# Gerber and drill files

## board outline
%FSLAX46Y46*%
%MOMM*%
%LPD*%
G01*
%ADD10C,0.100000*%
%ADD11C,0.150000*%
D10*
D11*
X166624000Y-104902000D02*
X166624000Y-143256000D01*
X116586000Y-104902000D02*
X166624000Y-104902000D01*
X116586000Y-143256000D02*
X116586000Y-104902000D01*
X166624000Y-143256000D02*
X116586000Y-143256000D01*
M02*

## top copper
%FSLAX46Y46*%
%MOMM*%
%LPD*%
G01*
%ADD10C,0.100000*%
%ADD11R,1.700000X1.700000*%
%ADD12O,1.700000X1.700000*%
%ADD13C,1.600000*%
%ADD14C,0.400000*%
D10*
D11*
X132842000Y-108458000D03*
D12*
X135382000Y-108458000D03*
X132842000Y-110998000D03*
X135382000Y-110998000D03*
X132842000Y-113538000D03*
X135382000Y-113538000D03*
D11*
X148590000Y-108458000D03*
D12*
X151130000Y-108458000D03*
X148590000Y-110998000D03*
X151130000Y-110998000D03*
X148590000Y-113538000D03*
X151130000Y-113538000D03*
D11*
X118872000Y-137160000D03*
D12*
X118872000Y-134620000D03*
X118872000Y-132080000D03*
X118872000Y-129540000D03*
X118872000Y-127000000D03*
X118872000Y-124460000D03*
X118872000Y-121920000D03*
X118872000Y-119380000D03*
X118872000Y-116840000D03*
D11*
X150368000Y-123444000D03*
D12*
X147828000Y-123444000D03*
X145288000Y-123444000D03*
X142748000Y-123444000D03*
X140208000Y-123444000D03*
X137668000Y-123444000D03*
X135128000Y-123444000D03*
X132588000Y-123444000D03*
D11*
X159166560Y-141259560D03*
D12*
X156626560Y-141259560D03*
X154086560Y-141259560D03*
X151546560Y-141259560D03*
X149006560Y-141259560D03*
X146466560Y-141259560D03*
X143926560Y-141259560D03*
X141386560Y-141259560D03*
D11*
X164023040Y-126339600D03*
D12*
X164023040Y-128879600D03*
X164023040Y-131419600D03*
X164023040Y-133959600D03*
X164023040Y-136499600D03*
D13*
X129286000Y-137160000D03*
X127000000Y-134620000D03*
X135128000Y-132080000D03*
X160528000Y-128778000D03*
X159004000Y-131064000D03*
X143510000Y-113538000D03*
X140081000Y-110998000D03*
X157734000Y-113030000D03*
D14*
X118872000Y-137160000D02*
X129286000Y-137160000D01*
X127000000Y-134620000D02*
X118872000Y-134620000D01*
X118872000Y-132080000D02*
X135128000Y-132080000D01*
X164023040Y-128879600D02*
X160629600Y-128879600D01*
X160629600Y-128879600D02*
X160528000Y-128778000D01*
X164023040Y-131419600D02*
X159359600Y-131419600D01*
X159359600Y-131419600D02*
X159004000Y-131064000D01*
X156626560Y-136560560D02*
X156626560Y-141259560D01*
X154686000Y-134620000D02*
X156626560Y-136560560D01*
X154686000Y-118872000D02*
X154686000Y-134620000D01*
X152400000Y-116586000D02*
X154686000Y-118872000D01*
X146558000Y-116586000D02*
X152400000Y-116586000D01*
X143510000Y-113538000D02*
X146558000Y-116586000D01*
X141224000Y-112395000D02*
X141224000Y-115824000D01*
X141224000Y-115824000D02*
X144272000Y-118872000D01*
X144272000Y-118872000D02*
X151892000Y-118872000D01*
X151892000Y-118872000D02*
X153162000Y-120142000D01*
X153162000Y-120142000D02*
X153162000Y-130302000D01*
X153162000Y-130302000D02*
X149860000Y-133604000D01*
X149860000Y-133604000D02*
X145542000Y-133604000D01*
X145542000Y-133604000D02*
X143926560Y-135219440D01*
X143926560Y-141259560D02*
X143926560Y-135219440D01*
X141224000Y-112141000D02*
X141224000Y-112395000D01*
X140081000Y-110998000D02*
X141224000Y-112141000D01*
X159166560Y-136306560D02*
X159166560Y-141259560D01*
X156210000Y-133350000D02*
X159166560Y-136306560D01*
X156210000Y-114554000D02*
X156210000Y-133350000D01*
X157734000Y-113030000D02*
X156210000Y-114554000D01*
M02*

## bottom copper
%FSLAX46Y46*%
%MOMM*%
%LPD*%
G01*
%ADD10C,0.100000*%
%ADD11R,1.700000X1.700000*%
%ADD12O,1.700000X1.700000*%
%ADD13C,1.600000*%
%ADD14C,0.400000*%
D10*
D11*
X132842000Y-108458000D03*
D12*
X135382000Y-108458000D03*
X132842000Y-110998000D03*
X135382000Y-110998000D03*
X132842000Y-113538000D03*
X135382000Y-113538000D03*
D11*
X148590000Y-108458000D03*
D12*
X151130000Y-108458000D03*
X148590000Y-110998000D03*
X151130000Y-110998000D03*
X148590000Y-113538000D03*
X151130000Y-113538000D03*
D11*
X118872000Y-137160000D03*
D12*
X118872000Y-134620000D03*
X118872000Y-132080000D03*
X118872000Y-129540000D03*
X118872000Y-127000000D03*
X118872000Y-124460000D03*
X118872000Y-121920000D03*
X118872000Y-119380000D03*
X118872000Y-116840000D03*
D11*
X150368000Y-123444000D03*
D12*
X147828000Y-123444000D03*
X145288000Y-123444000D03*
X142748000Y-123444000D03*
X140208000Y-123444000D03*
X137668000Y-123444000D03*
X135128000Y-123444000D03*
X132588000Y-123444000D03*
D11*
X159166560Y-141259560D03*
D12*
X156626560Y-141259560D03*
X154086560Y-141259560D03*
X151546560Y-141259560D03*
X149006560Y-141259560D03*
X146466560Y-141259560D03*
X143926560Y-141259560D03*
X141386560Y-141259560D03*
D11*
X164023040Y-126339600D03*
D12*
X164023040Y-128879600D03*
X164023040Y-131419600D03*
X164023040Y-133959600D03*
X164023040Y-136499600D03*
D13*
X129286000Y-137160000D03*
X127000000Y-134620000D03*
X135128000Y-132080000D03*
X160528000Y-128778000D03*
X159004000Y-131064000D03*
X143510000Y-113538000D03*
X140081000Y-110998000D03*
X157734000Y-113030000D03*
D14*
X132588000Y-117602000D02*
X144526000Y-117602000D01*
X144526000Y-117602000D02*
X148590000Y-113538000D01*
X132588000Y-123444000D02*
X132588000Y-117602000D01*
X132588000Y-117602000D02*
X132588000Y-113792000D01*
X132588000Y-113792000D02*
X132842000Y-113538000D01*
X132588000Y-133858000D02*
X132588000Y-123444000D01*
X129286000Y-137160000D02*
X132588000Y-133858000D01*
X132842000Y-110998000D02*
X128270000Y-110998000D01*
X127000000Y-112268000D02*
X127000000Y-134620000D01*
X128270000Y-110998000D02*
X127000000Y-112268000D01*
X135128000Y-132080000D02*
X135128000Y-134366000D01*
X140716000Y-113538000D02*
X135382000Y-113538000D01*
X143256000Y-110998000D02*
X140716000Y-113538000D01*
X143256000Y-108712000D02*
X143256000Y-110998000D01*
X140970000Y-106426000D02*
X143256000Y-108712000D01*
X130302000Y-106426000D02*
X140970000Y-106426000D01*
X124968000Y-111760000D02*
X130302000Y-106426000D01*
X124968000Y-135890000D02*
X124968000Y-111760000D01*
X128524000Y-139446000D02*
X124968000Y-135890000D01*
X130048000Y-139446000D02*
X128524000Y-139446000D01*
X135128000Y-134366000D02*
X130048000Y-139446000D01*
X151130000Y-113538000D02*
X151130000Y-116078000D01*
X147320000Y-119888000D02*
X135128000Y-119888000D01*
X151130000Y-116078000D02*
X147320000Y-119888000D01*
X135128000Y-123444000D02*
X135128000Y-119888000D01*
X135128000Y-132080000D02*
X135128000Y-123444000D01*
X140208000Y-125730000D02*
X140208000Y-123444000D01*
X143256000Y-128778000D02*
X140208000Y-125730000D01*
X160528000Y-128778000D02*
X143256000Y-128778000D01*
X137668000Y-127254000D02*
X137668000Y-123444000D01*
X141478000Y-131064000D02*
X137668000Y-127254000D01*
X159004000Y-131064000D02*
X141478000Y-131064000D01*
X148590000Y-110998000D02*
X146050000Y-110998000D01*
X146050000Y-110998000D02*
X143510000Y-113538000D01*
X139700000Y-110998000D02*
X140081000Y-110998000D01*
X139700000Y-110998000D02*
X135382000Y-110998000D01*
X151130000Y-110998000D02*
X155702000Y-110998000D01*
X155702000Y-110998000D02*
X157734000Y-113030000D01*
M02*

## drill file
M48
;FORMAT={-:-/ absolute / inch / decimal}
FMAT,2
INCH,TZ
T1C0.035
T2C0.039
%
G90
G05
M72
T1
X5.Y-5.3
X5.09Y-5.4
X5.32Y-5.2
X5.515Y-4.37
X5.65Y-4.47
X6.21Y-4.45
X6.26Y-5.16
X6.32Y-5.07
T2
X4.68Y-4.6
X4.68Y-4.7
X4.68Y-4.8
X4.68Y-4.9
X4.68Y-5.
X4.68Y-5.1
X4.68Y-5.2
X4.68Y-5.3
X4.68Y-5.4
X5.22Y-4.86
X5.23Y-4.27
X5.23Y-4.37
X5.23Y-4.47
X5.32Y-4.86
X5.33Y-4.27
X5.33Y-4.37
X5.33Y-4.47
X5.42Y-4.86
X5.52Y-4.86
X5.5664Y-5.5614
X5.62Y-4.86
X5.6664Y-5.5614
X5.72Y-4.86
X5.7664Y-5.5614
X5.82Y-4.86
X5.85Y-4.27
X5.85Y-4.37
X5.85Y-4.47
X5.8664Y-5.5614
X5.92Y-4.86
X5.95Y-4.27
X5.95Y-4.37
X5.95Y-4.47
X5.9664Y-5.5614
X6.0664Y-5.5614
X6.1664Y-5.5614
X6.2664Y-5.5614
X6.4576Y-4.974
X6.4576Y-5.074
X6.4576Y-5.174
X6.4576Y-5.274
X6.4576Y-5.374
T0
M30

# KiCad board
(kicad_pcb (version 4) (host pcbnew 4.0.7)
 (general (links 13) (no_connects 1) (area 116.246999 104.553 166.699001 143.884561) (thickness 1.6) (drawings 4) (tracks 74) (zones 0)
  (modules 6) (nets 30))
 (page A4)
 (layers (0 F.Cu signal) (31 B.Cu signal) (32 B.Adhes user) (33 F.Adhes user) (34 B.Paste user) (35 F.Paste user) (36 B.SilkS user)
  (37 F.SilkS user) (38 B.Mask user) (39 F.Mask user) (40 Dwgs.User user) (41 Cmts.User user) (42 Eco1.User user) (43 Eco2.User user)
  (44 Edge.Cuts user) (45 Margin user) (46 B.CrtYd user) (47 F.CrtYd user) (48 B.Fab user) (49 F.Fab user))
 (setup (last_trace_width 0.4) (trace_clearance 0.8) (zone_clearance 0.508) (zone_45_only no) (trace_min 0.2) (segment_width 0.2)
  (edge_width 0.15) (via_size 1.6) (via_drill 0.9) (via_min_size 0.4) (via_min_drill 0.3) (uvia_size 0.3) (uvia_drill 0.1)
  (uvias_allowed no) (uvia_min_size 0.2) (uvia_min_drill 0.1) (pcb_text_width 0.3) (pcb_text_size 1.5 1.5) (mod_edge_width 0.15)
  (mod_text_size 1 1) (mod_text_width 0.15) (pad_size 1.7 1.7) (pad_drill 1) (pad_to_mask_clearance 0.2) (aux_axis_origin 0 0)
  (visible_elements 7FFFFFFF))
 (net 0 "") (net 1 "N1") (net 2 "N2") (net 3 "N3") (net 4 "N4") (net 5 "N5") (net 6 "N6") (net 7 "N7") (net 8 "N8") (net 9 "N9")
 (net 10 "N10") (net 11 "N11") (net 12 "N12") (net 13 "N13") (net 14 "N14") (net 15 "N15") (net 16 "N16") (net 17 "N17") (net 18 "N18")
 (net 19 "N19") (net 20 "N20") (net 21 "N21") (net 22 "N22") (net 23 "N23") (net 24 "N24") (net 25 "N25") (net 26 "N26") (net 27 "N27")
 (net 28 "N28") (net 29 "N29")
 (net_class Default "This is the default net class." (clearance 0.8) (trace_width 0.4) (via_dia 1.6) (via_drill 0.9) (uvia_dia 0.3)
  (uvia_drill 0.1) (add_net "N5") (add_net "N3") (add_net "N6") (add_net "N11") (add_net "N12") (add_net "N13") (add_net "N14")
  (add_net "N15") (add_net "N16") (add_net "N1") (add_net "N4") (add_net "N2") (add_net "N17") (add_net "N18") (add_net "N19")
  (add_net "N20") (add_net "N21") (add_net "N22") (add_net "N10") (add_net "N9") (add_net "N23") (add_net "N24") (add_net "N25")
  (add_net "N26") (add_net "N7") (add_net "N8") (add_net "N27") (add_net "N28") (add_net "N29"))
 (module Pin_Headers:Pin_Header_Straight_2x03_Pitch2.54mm (layer F.Cu) (at 132.842 108.458)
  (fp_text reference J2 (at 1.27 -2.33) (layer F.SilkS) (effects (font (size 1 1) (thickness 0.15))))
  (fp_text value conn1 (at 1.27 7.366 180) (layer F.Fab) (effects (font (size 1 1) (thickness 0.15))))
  (pad 1 thru_hole rect (at 0 0) (size 1.7 1.7) (drill 1) (layers *.Cu *.Mask) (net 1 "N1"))
  (pad 6 thru_hole oval (at 2.54 0) (size 1.7 1.7) (drill 1) (layers *.Cu *.Mask) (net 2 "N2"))
  (pad 5 thru_hole oval (at 0 2.54) (size 1.7 1.7) (drill 1) (layers *.Cu *.Mask) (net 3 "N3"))
  (pad 2 thru_hole oval (at 2.54 2.54) (size 1.7 1.7) (drill 1) (layers *.Cu *.Mask) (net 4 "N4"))
  (pad 3 thru_hole oval (at 0 5.08) (size 1.7 1.7) (drill 1) (layers *.Cu *.Mask) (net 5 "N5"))
  (pad 4 thru_hole oval (at 2.54 5.08) (size 1.7 1.7) (drill 1) (layers *.Cu *.Mask) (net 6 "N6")))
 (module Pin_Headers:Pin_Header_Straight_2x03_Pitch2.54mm (layer F.Cu) (at 148.59 108.458)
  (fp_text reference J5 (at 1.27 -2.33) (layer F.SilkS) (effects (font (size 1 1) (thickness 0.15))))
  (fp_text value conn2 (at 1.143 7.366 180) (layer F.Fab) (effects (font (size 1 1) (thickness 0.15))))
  (pad 1 thru_hole rect (at 0 0) (size 1.7 1.7) (drill 1) (layers *.Cu *.Mask) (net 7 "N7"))
  (pad 6 thru_hole oval (at 2.54 0) (size 1.7 1.7) (drill 1) (layers *.Cu *.Mask) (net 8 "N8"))
  (pad 2 thru_hole oval (at 0 2.54) (size 1.7 1.7) (drill 1) (layers *.Cu *.Mask) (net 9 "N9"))
  (pad 5 thru_hole oval (at 2.54 2.54) (size 1.7 1.7) (drill 1) (layers *.Cu *.Mask) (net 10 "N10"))
  (pad 3 thru_hole oval (at 0 5.08) (size 1.7 1.7) (drill 1) (layers *.Cu *.Mask) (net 5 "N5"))
  (pad 4 thru_hole oval (at 2.54 5.08) (size 1.7 1.7) (drill 1) (layers *.Cu *.Mask) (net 6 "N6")))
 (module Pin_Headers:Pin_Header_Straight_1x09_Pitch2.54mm (layer F.Cu) (at 118.872 137.16 180)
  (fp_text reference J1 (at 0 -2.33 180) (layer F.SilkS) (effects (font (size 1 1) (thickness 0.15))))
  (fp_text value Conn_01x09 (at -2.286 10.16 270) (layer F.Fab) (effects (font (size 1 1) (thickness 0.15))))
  (pad 1 thru_hole rect (at 0 0 180) (size 1.7 1.7) (drill 1) (layers *.Cu *.Mask) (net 5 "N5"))
  (pad 2 thru_hole oval (at 0 2.54 180) (size 1.7 1.7) (drill 1) (layers *.Cu *.Mask) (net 3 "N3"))
  (pad 3 thru_hole oval (at 0 5.08 180) (size 1.7 1.7) (drill 1) (layers *.Cu *.Mask) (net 6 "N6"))
  (pad 4 thru_hole oval (at 0 7.62 180) (size 1.7 1.7) (drill 1) (layers *.Cu *.Mask) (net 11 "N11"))
  (pad 5 thru_hole oval (at 0 10.16 180) (size 1.7 1.7) (drill 1) (layers *.Cu *.Mask) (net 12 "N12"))
  (pad 6 thru_hole oval (at 0 12.7 180) (size 1.7 1.7) (drill 1) (layers *.Cu *.Mask) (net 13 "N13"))
  (pad 7 thru_hole oval (at 0 15.24 180) (size 1.7 1.7) (drill 1) (layers *.Cu *.Mask) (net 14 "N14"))
  (pad 8 thru_hole oval (at 0 17.78 180) (size 1.7 1.7) (drill 1) (layers *.Cu *.Mask) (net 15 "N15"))
  (pad 9 thru_hole oval (at 0 20.32 180) (size 1.7 1.7) (drill 1) (layers *.Cu *.Mask) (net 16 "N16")))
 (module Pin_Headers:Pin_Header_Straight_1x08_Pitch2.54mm (layer F.Cu) (at 150.368 123.444 270)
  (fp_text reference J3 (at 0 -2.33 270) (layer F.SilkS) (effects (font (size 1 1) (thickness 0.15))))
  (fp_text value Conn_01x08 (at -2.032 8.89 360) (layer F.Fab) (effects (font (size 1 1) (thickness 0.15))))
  (pad 1 thru_hole rect (at 0 0 270) (size 1.7 1.7) (drill 1) (layers *.Cu *.Mask) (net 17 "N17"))
  (pad 2 thru_hole oval (at 0 2.54 270) (size 1.7 1.7) (drill 1) (layers *.Cu *.Mask) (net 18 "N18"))
  (pad 3 thru_hole oval (at 0 5.08 270) (size 1.7 1.7) (drill 1) (layers *.Cu *.Mask) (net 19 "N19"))
  (pad 4 thru_hole oval (at 0 7.62 270) (size 1.7 1.7) (drill 1) (layers *.Cu *.Mask) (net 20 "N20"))
  (pad 5 thru_hole oval (at 0 10.16 270) (size 1.7 1.7) (drill 1) (layers *.Cu *.Mask) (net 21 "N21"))
  (pad 6 thru_hole oval (at 0 12.7 270) (size 1.7 1.7) (drill 1) (layers *.Cu *.Mask) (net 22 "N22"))
  (pad 7 thru_hole oval (at 0 15.24 270) (size 1.7 1.7) (drill 1) (layers *.Cu *.Mask) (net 6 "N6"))
  (pad 8 thru_hole oval (at 0 17.78 270) (size 1.7 1.7) (drill 1) (layers *.Cu *.Mask) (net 5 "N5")))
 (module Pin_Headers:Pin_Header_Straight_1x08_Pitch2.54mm (layer F.Cu) (at 159.16656 141.25956 270)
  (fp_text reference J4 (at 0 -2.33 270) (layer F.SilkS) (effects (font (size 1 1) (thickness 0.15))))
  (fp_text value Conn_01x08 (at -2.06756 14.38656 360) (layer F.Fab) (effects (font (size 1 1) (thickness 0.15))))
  (pad 1 thru_hole rect (at 0 0 270) (size 1.7 1.7) (drill 1) (layers *.Cu *.Mask) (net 10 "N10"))
  (pad 2 thru_hole oval (at 0 2.54 270) (size 1.7 1.7) (drill 1) (layers *.Cu *.Mask) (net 9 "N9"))
  (pad 3 thru_hole oval (at 0 5.08 270) (size 1.7 1.7) (drill 1) (layers *.Cu *.Mask) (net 6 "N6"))
  (pad 4 thru_hole oval (at 0 7.62 270) (size 1.7 1.7) (drill 1) (layers *.Cu *.Mask) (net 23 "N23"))
  (pad 5 thru_hole oval (at 0 10.16 270) (size 1.7 1.7) (drill 1) (layers *.Cu *.Mask) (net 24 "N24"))
  (pad 6 thru_hole oval (at 0 12.7 270) (size 1.7 1.7) (drill 1) (layers *.Cu *.Mask) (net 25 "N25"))
  (pad 7 thru_hole oval (at 0 15.24 270) (size 1.7 1.7) (drill 1) (layers *.Cu *.Mask) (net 4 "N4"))
  (pad 8 thru_hole oval (at 0 17.78 270) (size 1.7 1.7) (drill 1) (layers *.Cu *.Mask) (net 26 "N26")))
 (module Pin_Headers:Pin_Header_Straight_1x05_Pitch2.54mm (layer F.Cu) (at 164.02304 126.3396)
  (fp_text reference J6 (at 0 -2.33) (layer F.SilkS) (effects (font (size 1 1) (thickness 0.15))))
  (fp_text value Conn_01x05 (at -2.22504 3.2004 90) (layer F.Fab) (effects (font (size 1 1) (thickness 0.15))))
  (pad 1 thru_hole rect (at 0 0) (size 1.7 1.7) (drill 1) (layers *.Cu *.Mask) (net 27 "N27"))
  (pad 2 thru_hole oval (at 0 2.54) (size 1.7 1.7) (drill 1) (layers *.Cu *.Mask) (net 21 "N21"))
  (pad 3 thru_hole oval (at 0 5.08) (size 1.7 1.7) (drill 1) (layers *.Cu *.Mask) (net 22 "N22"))
  (pad 4 thru_hole oval (at 0 7.62) (size 1.7 1.7) (drill 1) (layers *.Cu *.Mask) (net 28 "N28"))
  (pad 5 thru_hole oval (at 0 10.16) (size 1.7 1.7) (drill 1) (layers *.Cu *.Mask) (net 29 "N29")))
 (gr_line (start 166.624 104.902) (end 166.624 143.256) (angle 90) (layer Edge.Cuts) (width 0.15))
 (gr_line (start 116.586 104.902) (end 166.624 104.902) (angle 90) (layer Edge.Cuts) (width 0.15))
 (gr_line (start 116.586 143.256) (end 116.586 104.902) (angle 90) (layer Edge.Cuts) (width 0.15))
 (gr_line (start 166.624 143.256) (end 116.586 143.256) (angle 90) (layer Edge.Cuts) (width 0.15))
 (segment (start 132.588 117.602) (end 144.526 117.602) (width 0.4) (layer B.Cu) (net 5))
 (segment (start 144.526 117.602) (end 148.59 113.538) (width 0.4) (layer B.Cu) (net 5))
 (segment (start 132.588 123.444) (end 132.588 117.602) (width 0.4) (layer B.Cu) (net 5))
 (segment (start 132.588 117.602) (end 132.588 113.792) (width 0.4) (layer B.Cu) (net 5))
 (segment (start 132.588 113.792) (end 132.842 113.538) (width 0.4) (layer B.Cu) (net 5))
 (segment (start 118.872 137.16) (end 129.286 137.16) (width 0.4) (layer F.Cu) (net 5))
 (segment (start 132.588 133.858) (end 132.588 123.444) (width 0.4) (layer B.Cu) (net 5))
 (segment (start 129.286 137.16) (end 132.588 133.858) (width 0.4) (layer B.Cu) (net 5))
 (via (at 129.286 137.16) (size 1.6) (drill 0.9) (layers F.Cu B.Cu) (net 5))
 (segment (start 132.842 110.998) (end 128.27 110.998) (width 0.4) (layer B.Cu) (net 3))
 (segment (start 127 134.62) (end 118.872 134.62) (width 0.4) (layer F.Cu) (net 3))
 (via (at 127 134.62) (size 1.6) (drill 0.9) (layers F.Cu B.Cu) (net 3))
 (segment (start 127 112.268) (end 127 134.62) (width 0.4) (layer B.Cu) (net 3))
 (segment (start 128.27 110.998) (end 127 112.268) (width 0.4) (layer B.Cu) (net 3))
 (segment (start 135.128 132.08) (end 135.128 134.366) (width 0.4) (layer B.Cu) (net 6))
 (segment (start 140.716 113.538) (end 135.382 113.538) (width 0.4) (layer B.Cu) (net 6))
 (segment (start 143.256 110.998) (end 140.716 113.538) (width 0.4) (layer B.Cu) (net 6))
 (segment (start 143.256 108.712) (end 143.256 110.998) (width 0.4) (layer B.Cu) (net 6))
 (segment (start 140.97 106.426) (end 143.256 108.712) (width 0.4) (layer B.Cu) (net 6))
 (segment (start 130.302 106.426) (end 140.97 106.426) (width 0.4) (layer B.Cu) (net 6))
 (segment (start 124.968 111.76) (end 130.302 106.426) (width 0.4) (layer B.Cu) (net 6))
 (segment (start 124.968 135.89) (end 124.968 111.76) (width 0.4) (layer B.Cu) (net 6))
 (segment (start 128.524 139.446) (end 124.968 135.89) (width 0.4) (layer B.Cu) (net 6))
 (segment (start 130.048 139.446) (end 128.524 139.446) (width 0.4) (layer B.Cu) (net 6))
 (segment (start 135.128 134.366) (end 130.048 139.446) (width 0.4) (layer B.Cu) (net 6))
 (segment (start 151.13 113.538) (end 151.13 116.078) (width 0.4) (layer B.Cu) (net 6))
 (segment (start 147.32 119.888) (end 135.128 119.888) (width 0.4) (layer B.Cu) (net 6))
 (segment (start 151.13 116.078) (end 147.32 119.888) (width 0.4) (layer B.Cu) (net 6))
 (segment (start 135.128 123.444) (end 135.128 119.888) (width 0.4) (layer B.Cu) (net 6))
 (segment (start 118.872 132.08) (end 135.128 132.08) (width 0.4) (layer F.Cu) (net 6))
 (segment (start 135.128 132.08) (end 135.128 123.444) (width 0.4) (layer B.Cu) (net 6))
 (via (at 135.128 132.08) (size 1.6) (drill 0.9) (layers F.Cu B.Cu) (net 6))
 (segment (start 164.02304 128.8796) (end 160.6296 128.8796) (width 0.4) (layer F.Cu) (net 21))
 (segment (start 140.208 125.73) (end 140.208 123.444) (width 0.4) (layer B.Cu) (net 21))
 (segment (start 143.256 128.778) (end 140.208 125.73) (width 0.4) (layer B.Cu) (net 21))
 (segment (start 160.528 128.778) (end 143.256 128.778) (width 0.4) (layer B.Cu) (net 21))
 (via (at 160.528 128.778) (size 1.6) (drill 0.9) (layers F.Cu B.Cu) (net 21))
 (segment (start 160.6296 128.8796) (end 160.528 128.778) (width 0.4) (layer F.Cu) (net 21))
 (segment (start 164.02304 131.4196) (end 159.3596 131.4196) (width 0.4) (layer F.Cu) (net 22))
 (segment (start 137.668 127.254) (end 137.668 123.444) (width 0.4) (layer B.Cu) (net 22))
 (segment (start 141.478 131.064) (end 137.668 127.254) (width 0.4) (layer B.Cu) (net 22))
 (segment (start 159.004 131.064) (end 141.478 131.064) (width 0.4) (layer B.Cu) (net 22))
 (via (at 159.004 131.064) (size 1.6) (drill 0.9) (layers F.Cu B.Cu) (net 22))
 (segment (start 159.3596 131.4196) (end 159.004 131.064) (width 0.4) (layer F.Cu) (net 22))
 (segment (start 148.59 110.998) (end 146.05 110.998) (width 0.4) (layer B.Cu) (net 9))
 (segment (start 156.62656 136.56056) (end 156.62656 141.25956) (width 0.4) (layer F.Cu) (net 9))
 (segment (start 154.686 134.62) (end 156.62656 136.56056) (width 0.4) (layer F.Cu) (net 9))
 (segment (start 154.686 118.872) (end 154.686 134.62) (width 0.4) (layer F.Cu) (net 9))
 (segment (start 152.4 116.586) (end 154.686 118.872) (width 0.4) (layer F.Cu) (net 9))
 (segment (start 146.558 116.586) (end 152.4 116.586) (width 0.4) (layer F.Cu) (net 9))
 (segment (start 143.51 113.538) (end 146.558 116.586) (width 0.4) (layer F.Cu) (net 9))
 (via (at 143.51 113.538) (size 1.6) (drill 0.9) (layers F.Cu B.Cu) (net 9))
 (segment (start 146.05 110.998) (end 143.51 113.538) (width 0.4) (layer B.Cu) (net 9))
 (segment (start 139.7 110.998) (end 140.081 110.998) (width 0.4) (layer B.Cu) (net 4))
 (segment (start 141.224 112.395) (end 141.224 115.824) (width 0.4) (layer F.Cu) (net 4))
 (segment (start 141.224 115.824) (end 144.272 118.872) (width 0.4) (layer F.Cu) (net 4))
 (segment (start 144.272 118.872) (end 151.892 118.872) (width 0.4) (layer F.Cu) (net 4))
 (segment (start 151.892 118.872) (end 153.162 120.142) (width 0.4) (layer F.Cu) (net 4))
 (segment (start 153.162 120.142) (end 153.162 130.302) (width 0.4) (layer F.Cu) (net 4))
 (segment (start 153.162 130.302) (end 149.86 133.604) (width 0.4) (layer F.Cu) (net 4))
 (segment (start 149.86 133.604) (end 145.542 133.604) (width 0.4) (layer F.Cu) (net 4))
 (segment (start 145.542 133.604) (end 143.92656 135.21944) (width 0.4) (layer F.Cu) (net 4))
 (segment (start 143.92656 141.25956) (end 143.92656 135.21944) (width 0.4) (layer F.Cu) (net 4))
 (segment (start 139.7 110.998) (end 135.382 110.998) (width 0.4) (layer B.Cu) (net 4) (status 800000))
 (segment (start 141.224 112.141) (end 141.224 112.395) (width 0.4) (layer F.Cu) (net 4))
 (segment (start 140.081 110.998) (end 141.224 112.141) (width 0.4) (layer F.Cu) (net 4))
 (via (at 140.081 110.998) (size 1.6) (drill 0.9) (layers F.Cu B.Cu) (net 4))
 (segment (start 151.13 110.998) (end 155.702 110.998) (width 0.4) (layer B.Cu) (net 10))
 (segment (start 159.16656 136.30656) (end 159.16656 141.25956) (width 0.4) (layer F.Cu) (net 10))
 (segment (start 156.21 133.35) (end 159.16656 136.30656) (width 0.4) (layer F.Cu) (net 10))
 (segment (start 156.21 114.554) (end 156.21 133.35) (width 0.4) (layer F.Cu) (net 10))
 (segment (start 157.734 113.03) (end 156.21 114.554) (width 0.4) (layer F.Cu) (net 10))
 (via (at 157.734 113.03) (size 1.6) (drill 0.9) (layers F.Cu B.Cu) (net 10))
 (segment (start 155.702 110.998) (end 157.734 113.03) (width 0.4) (layer B.Cu) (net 10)))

